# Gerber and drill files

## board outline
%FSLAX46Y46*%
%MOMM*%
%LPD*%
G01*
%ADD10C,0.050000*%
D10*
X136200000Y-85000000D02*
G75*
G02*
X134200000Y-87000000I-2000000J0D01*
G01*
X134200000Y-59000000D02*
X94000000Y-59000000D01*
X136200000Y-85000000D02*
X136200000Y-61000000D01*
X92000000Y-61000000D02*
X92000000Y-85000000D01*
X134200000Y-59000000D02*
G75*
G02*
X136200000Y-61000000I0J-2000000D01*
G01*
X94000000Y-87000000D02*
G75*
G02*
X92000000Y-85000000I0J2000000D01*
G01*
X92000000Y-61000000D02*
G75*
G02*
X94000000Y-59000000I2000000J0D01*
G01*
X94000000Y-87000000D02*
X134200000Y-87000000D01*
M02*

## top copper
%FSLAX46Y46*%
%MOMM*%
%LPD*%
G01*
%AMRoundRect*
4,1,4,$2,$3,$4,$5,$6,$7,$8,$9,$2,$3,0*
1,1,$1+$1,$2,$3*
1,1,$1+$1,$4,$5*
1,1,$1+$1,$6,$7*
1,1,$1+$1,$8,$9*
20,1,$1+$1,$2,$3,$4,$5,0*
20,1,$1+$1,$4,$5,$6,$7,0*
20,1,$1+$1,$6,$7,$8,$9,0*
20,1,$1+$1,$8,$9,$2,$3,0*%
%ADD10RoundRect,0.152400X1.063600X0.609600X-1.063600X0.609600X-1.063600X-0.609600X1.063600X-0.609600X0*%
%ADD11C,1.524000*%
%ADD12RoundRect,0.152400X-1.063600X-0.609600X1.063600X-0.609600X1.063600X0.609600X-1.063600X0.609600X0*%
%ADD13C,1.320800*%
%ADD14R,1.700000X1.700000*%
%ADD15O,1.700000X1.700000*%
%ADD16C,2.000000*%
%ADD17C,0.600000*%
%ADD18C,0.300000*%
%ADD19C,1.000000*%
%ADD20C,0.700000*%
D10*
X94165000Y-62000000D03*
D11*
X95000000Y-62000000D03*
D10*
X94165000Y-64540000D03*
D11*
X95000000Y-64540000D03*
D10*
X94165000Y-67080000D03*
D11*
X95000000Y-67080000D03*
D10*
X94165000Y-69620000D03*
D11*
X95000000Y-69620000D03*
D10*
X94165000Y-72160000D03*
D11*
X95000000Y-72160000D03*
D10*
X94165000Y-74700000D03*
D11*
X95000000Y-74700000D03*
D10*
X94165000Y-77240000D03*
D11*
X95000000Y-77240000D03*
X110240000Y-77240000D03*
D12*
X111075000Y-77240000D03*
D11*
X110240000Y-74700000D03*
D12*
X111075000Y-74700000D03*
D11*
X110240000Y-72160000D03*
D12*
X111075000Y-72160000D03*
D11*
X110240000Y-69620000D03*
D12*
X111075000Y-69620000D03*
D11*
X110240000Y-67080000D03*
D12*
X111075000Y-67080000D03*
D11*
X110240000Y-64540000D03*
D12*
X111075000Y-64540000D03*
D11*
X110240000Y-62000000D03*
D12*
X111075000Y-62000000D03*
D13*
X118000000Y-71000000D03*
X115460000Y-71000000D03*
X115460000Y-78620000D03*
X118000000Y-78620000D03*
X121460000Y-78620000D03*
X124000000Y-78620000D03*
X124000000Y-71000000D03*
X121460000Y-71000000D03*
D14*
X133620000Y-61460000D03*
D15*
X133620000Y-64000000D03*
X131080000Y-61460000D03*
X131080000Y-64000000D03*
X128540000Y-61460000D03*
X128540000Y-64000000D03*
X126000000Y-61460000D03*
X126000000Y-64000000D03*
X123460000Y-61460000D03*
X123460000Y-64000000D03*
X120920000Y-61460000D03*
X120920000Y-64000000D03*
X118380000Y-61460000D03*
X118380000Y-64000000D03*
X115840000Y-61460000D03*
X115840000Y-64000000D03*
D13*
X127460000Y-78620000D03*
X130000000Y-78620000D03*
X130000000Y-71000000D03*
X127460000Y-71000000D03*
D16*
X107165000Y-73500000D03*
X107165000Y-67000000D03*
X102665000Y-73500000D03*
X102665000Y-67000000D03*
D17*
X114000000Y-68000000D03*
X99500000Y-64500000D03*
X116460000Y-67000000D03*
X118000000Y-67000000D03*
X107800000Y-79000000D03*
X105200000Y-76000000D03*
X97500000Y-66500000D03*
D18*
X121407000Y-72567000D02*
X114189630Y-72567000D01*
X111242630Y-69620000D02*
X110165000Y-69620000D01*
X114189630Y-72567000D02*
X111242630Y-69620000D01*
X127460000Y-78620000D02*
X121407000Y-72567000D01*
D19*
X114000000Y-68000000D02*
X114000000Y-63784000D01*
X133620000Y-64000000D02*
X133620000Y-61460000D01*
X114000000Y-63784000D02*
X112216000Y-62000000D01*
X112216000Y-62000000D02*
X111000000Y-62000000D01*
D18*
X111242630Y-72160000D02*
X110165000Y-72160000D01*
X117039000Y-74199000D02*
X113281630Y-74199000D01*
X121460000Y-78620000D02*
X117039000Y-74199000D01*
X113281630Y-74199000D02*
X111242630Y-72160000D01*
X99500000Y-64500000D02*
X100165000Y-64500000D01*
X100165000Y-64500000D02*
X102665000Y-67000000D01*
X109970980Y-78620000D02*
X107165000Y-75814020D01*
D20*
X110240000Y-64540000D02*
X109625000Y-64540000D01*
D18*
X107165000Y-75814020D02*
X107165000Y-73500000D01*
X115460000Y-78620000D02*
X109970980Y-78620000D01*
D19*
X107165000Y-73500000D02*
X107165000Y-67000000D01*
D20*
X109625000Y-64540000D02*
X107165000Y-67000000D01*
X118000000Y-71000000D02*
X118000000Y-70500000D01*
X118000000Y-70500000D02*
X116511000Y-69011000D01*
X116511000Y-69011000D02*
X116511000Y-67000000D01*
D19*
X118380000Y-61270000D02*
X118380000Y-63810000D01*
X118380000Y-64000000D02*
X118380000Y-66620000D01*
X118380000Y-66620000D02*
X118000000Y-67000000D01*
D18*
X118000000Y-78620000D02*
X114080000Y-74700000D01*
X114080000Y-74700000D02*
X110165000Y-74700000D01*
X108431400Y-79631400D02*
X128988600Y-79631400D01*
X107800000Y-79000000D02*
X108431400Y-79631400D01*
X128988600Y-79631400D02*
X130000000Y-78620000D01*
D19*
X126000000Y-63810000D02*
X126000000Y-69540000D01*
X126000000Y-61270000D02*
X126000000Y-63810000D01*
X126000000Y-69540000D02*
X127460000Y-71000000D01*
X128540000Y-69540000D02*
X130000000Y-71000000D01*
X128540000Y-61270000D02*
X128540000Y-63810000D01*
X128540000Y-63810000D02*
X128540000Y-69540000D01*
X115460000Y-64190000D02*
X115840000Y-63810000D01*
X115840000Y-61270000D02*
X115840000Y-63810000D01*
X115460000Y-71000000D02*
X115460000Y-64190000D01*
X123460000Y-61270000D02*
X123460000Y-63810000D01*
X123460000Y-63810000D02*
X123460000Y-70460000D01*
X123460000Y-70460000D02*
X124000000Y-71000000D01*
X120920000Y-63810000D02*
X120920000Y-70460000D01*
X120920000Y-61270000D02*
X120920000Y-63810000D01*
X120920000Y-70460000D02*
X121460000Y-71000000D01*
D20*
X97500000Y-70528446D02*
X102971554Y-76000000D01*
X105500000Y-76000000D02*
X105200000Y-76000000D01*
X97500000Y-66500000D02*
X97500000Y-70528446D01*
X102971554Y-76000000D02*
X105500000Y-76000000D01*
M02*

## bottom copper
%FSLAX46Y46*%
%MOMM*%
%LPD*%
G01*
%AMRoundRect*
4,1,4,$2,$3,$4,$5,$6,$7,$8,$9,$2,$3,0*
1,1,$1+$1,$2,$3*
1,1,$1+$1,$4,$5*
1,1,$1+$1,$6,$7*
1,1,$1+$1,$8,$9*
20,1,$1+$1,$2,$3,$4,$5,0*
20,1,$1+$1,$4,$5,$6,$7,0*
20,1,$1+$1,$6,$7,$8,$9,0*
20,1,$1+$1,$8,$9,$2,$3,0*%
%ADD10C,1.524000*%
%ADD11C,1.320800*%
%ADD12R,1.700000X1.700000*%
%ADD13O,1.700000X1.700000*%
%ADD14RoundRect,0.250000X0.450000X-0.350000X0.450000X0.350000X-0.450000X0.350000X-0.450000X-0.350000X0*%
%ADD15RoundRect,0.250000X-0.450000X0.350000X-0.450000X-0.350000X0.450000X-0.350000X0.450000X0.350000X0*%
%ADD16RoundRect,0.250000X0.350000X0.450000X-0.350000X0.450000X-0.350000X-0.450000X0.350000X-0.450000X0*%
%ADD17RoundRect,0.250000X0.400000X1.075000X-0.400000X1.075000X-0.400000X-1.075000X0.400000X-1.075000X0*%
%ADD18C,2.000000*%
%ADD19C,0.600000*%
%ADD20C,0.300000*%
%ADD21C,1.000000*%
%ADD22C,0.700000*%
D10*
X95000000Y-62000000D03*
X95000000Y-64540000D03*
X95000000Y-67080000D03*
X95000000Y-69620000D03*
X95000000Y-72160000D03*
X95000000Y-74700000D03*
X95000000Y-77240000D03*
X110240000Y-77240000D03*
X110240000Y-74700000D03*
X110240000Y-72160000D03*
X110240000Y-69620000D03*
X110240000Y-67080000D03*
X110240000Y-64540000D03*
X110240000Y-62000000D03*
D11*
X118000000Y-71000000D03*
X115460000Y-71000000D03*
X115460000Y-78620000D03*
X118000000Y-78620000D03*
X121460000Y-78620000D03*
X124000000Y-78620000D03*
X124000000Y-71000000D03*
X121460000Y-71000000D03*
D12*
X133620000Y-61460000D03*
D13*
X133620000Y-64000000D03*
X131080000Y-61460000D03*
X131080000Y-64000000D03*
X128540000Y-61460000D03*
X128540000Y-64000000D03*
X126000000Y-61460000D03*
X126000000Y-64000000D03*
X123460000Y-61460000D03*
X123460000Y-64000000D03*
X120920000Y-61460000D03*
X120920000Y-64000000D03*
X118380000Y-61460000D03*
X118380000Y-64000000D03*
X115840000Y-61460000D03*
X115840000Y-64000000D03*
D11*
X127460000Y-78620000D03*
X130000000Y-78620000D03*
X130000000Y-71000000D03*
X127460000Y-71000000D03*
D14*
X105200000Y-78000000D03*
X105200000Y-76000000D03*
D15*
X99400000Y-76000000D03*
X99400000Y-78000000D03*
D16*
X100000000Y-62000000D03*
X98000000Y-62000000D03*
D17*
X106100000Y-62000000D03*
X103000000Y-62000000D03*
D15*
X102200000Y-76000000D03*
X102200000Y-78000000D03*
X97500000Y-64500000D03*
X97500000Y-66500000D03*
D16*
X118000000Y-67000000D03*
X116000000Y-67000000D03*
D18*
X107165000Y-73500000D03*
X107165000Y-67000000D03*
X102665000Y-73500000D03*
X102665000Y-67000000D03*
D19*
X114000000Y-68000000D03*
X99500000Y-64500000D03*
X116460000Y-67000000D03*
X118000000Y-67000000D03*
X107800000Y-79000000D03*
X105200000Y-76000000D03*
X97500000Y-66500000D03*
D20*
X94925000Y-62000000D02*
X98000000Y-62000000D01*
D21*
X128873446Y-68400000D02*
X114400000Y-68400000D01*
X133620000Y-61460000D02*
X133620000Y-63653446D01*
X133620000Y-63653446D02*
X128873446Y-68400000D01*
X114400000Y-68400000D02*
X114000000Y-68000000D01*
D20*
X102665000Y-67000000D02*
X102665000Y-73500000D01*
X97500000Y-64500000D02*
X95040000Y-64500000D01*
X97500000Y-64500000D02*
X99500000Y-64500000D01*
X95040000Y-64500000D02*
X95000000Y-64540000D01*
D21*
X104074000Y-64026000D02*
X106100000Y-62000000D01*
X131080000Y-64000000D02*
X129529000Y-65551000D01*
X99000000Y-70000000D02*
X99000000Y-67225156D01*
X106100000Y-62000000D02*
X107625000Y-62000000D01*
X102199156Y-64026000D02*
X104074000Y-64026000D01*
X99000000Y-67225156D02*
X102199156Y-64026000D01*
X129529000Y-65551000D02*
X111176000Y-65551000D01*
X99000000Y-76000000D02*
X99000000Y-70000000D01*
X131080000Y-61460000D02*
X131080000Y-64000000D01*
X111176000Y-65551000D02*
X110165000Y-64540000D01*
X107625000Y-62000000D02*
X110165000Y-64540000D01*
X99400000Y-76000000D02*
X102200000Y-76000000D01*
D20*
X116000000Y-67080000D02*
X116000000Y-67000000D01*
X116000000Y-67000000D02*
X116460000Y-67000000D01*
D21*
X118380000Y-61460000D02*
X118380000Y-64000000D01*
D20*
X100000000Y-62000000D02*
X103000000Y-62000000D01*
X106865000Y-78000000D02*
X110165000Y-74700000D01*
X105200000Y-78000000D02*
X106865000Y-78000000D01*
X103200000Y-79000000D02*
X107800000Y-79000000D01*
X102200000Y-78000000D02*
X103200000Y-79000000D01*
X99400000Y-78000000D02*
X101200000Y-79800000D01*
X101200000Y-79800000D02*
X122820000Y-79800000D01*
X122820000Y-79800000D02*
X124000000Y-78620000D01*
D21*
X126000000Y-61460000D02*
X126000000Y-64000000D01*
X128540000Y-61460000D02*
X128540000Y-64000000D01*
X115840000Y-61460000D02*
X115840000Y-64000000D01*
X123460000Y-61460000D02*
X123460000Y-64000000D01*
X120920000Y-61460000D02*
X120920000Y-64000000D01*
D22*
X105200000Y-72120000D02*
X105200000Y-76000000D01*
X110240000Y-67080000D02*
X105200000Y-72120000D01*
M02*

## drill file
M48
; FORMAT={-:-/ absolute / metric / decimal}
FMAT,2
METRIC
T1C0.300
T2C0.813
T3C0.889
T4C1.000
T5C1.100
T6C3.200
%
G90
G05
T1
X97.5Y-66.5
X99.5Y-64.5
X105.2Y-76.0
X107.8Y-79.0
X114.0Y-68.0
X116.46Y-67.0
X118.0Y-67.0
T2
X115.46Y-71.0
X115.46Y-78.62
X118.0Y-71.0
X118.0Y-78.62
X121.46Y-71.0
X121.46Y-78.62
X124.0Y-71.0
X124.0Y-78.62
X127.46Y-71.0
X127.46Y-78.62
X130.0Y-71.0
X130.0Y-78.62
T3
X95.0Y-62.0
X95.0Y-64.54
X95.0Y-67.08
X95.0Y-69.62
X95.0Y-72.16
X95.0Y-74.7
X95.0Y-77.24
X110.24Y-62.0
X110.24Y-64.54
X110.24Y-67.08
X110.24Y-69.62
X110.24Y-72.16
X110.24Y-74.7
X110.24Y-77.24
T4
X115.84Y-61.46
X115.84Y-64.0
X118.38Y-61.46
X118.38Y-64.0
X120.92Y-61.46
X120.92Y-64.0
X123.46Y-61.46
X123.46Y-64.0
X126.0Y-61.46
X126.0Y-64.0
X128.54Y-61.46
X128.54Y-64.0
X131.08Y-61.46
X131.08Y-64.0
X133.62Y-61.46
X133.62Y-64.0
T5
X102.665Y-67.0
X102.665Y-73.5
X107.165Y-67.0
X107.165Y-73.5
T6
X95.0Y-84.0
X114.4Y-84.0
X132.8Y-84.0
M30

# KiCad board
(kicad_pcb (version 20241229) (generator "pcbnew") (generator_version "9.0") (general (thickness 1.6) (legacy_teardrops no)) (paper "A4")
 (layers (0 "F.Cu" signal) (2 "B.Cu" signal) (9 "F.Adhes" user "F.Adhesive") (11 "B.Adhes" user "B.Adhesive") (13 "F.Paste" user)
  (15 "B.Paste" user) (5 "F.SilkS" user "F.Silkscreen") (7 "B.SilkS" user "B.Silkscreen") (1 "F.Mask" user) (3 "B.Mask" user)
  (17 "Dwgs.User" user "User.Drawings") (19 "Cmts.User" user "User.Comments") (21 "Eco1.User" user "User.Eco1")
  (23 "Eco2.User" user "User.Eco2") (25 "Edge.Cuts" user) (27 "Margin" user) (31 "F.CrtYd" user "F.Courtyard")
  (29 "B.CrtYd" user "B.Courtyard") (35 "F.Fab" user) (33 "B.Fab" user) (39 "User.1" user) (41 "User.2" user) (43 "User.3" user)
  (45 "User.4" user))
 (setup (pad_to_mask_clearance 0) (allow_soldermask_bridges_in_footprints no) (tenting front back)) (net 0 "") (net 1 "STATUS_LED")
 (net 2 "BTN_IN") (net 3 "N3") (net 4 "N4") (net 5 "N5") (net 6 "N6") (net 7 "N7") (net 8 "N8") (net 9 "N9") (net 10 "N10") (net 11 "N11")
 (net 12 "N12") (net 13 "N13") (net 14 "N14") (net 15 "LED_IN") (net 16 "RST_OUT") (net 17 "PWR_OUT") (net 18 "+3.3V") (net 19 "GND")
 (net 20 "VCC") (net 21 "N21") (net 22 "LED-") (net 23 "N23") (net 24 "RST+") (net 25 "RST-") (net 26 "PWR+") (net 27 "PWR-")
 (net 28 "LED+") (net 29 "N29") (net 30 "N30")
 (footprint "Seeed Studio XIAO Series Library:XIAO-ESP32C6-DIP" (layer "F.Cu") (at 102.665 69.62)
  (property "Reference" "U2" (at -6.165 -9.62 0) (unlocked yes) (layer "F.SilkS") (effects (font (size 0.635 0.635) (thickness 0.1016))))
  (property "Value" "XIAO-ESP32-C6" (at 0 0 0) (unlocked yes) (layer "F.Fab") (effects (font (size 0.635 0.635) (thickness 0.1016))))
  (pad "1" smd roundrect (at -8.5 -7.62 180) (size 2.432 1.524) (layers "F.Cu" "F.Mask") (roundrect_rratio 0.1) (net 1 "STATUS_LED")
   (thermal_bridge_angle 45))
  (pad "1" thru_hole circle (at -7.665 -7.62 180) (size 1.524 1.524) (drill 0.889) (layers "*.Cu" "*.Mask") (remove_unused_layers no)
   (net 1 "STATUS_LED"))
  (pad "2" smd roundrect (at -8.5 -5.08 180) (size 2.432 1.524) (layers "F.Cu" "F.Mask") (roundrect_rratio 0.1) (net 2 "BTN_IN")
   (thermal_bridge_angle 45))
  (pad "2" thru_hole circle (at -7.665 -5.08 180) (size 1.524 1.524) (drill 0.889) (layers "*.Cu" "*.Mask") (remove_unused_layers no)
   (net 2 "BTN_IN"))
  (pad "3" smd roundrect (at -8.5 -2.54 180) (size 2.432 1.524) (layers "F.Cu" "F.Mask") (roundrect_rratio 0.1) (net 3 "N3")
   (thermal_bridge_angle 45))
  (pad "3" thru_hole circle (at -7.665 -2.54 180) (size 1.524 1.524) (drill 0.889) (layers "*.Cu" "*.Mask") (remove_unused_layers no)
   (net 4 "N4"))
  (pad "4" smd roundrect (at -8.5 0 180) (size 2.432 1.524) (layers "F.Cu" "F.Mask") (roundrect_rratio 0.1) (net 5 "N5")
   (thermal_bridge_angle 45))
  (pad "4" thru_hole circle (at -7.665 0 180) (size 1.524 1.524) (drill 0.889) (layers "*.Cu" "*.Mask") (remove_unused_layers no)
   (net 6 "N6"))
  (pad "5" smd roundrect (at -8.5 2.54 180) (size 2.432 1.524) (layers "F.Cu" "F.Mask") (roundrect_rratio 0.1) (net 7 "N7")
   (thermal_bridge_angle 45))
  (pad "5" thru_hole circle (at -7.665 2.54 180) (size 1.524 1.524) (drill 0.889) (layers "*.Cu" "*.Mask") (remove_unused_layers no)
   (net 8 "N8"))
  (pad "6" smd roundrect (at -8.5 5.08 180) (size 2.432 1.524) (layers "F.Cu" "F.Mask") (roundrect_rratio 0.1) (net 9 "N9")
   (thermal_bridge_angle 45))
  (pad "6" thru_hole circle (at -7.665 5.08 180) (size 1.524 1.524) (drill 0.889) (layers "*.Cu" "*.Mask") (remove_unused_layers no)
   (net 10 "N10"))
  (pad "7" smd roundrect (at -8.5 7.62 180) (size 2.432 1.524) (layers "F.Cu" "F.Mask") (roundrect_rratio 0.1) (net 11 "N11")
   (thermal_bridge_angle 45))
  (pad "7" thru_hole circle (at -7.665 7.62 180) (size 1.524 1.524) (drill 0.889) (layers "*.Cu" "*.Mask") (remove_unused_layers no)
   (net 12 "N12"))
  (pad "8" thru_hole circle (at 7.575 7.62) (size 1.524 1.524) (drill 0.889) (layers "*.Cu" "*.Mask") (remove_unused_layers no)
   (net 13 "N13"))
  (pad "8" smd roundrect (at 8.41 7.62) (size 2.432 1.524) (layers "F.Cu" "F.Mask") (roundrect_rratio 0.1) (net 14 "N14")
   (thermal_bridge_angle 45))
  (pad "9" thru_hole circle (at 7.575 5.08) (size 1.524 1.524) (drill 0.889) (layers "*.Cu" "*.Mask") (remove_unused_layers no)
   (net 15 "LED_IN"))
  (pad "9" smd roundrect (at 8.41 5.08) (size 2.432 1.524) (layers "F.Cu" "F.Mask") (roundrect_rratio 0.1) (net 15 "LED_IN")
   (thermal_bridge_angle 45))
  (pad "10" thru_hole circle (at 7.575 2.54) (size 1.524 1.524) (drill 0.889) (layers "*.Cu" "*.Mask") (remove_unused_layers no)
   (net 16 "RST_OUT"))
  (pad "10" smd roundrect (at 8.41 2.54) (size 2.432 1.524) (layers "F.Cu" "F.Mask") (roundrect_rratio 0.1) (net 16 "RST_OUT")
   (thermal_bridge_angle 45))
  (pad "11" thru_hole circle (at 7.575 0) (size 1.524 1.524) (drill 0.889) (layers "*.Cu" "*.Mask") (remove_unused_layers no)
   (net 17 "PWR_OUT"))
  (pad "11" smd roundrect (at 8.41 0) (size 2.432 1.524) (layers "F.Cu" "F.Mask") (roundrect_rratio 0.1) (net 17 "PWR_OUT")
   (thermal_bridge_angle 45))
  (pad "12" thru_hole circle (at 7.575 -2.54) (size 1.524 1.524) (drill 0.889) (layers "*.Cu" "*.Mask") (remove_unused_layers no)
   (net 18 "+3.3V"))
  (pad "12" smd roundrect (at 8.41 -2.54) (size 2.432 1.524) (layers "F.Cu" "F.Mask") (roundrect_rratio 0.1) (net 18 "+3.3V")
   (thermal_bridge_angle 45))
  (pad "13" thru_hole circle (at 7.575 -5.08) (size 1.524 1.524) (drill 0.889) (layers "*.Cu" "*.Mask") (remove_unused_layers no)
   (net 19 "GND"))
  (pad "13" smd roundrect (at 8.41 -5.08) (size 2.432 1.524) (layers "F.Cu" "F.Mask") (roundrect_rratio 0.1) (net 19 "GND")
   (thermal_bridge_angle 45))
  (pad "14" thru_hole circle (at 7.575 -7.62) (size 1.524 1.524) (drill 0.889) (layers "*.Cu" "*.Mask") (remove_unused_layers no)
   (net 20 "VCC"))
  (pad "14" smd roundrect (at 8.41 -7.62) (size 2.432 1.524) (layers "F.Cu" "F.Mask") (roundrect_rratio 0.1) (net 20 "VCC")
   (thermal_bridge_angle 45)))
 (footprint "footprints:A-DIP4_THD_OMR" (layer "F.Cu") (at 118 71 -90)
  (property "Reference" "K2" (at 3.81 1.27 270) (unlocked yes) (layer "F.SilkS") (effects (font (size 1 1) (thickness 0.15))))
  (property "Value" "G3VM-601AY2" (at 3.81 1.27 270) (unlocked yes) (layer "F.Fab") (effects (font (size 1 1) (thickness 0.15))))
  (pad "1" thru_hole circle (at 0 0 270) (size 1.3208 1.3208) (drill 0.8128) (layers "*.Cu" "*.Mask") (remove_unused_layers no)
   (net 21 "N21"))
  (pad "2" thru_hole circle (at 0 2.54 270) (size 1.3208 1.3208) (drill 0.8128) (layers "*.Cu" "*.Mask") (remove_unused_layers no)
   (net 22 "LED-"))
  (pad "3" thru_hole circle (at 7.62 2.54 270) (size 1.3208 1.3208) (drill 0.8128) (layers "*.Cu" "*.Mask") (remove_unused_layers no)
   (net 19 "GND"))
  (pad "4" thru_hole circle (at 7.62 0 270) (size 1.3208 1.3208) (drill 0.8128) (layers "*.Cu" "*.Mask") (remove_unused_layers no)
   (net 15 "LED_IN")))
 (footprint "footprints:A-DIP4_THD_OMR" (layer "F.Cu") (at 121.46 78.62 90)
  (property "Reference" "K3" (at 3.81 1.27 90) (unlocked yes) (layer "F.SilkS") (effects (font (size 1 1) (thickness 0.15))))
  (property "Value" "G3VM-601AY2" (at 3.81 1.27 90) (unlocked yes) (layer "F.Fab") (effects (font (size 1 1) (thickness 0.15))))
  (pad "1" thru_hole circle (at 0 0 90) (size 1.3208 1.3208) (drill 0.8128) (layers "*.Cu" "*.Mask") (remove_unused_layers no)
   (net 16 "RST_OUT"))
  (pad "2" thru_hole circle (at 0 2.54 90) (size 1.3208 1.3208) (drill 0.8128) (layers "*.Cu" "*.Mask") (remove_unused_layers no)
   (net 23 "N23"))
  (pad "3" thru_hole circle (at 7.62 2.54 90) (size 1.3208 1.3208) (drill 0.8128) (layers "*.Cu" "*.Mask") (remove_unused_layers no)
   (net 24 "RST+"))
  (pad "4" thru_hole circle (at 7.62 0 90) (size 1.3208 1.3208) (drill 0.8128) (layers "*.Cu" "*.Mask") (remove_unused_layers no)
   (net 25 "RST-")))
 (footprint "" (layer "F.Cu") (at 132.8 84)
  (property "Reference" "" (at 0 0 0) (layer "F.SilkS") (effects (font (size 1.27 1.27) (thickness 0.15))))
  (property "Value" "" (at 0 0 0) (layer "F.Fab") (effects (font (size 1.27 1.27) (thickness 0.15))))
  (pad "" np_thru_hole circle (at 0 0) (size 3.2 3.2) (drill 3.2) (layers "*.Cu" "*.Mask")))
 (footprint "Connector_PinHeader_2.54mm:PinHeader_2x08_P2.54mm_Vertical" (layer "F.Cu") (at 133.62 61.46 -90)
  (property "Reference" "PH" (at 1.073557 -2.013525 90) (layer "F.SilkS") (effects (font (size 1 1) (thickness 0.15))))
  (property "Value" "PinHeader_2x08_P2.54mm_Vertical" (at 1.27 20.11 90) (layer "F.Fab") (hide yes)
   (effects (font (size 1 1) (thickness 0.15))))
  (pad "1" thru_hole rect (at 0 0 270) (size 1.7 1.7) (drill 1) (layers "*.Cu" "*.Mask") (remove_unused_layers no) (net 20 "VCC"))
  (pad "2" thru_hole oval (at 2.54 0 270) (size 1.7 1.7) (drill 1) (layers "*.Cu" "*.Mask") (remove_unused_layers no) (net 20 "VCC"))
  (pad "3" thru_hole oval (at 0 2.54 270) (size 1.7 1.7) (drill 1) (layers "*.Cu" "*.Mask") (remove_unused_layers no) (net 19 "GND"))
  (pad "4" thru_hole oval (at 2.54 2.54 270) (size 1.7 1.7) (drill 1) (layers "*.Cu" "*.Mask") (remove_unused_layers no) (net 19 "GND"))
  (pad "5" thru_hole oval (at 0 5.08 270) (size 1.7 1.7) (drill 1) (layers "*.Cu" "*.Mask") (remove_unused_layers no) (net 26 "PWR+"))
  (pad "6" thru_hole oval (at 2.54 5.08 270) (size 1.7 1.7) (drill 1) (layers "*.Cu" "*.Mask") (remove_unused_layers no) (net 26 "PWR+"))
  (pad "7" thru_hole oval (at 0 7.62 270) (size 1.7 1.7) (drill 1) (layers "*.Cu" "*.Mask") (remove_unused_layers no) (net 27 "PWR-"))
  (pad "8" thru_hole oval (at 2.54 7.62 270) (size 1.7 1.7) (drill 1) (layers "*.Cu" "*.Mask") (remove_unused_layers no) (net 27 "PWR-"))
  (pad "9" thru_hole oval (at 0 10.16 270) (size 1.7 1.7) (drill 1) (layers "*.Cu" "*.Mask") (remove_unused_layers no) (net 24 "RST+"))
  (pad "10" thru_hole oval (at 2.54 10.16 270) (size 1.7 1.7) (drill 1) (layers "*.Cu" "*.Mask") (remove_unused_layers no) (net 24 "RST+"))
  (pad "11" thru_hole oval (at 0 12.7 270) (size 1.7 1.7) (drill 1) (layers "*.Cu" "*.Mask") (remove_unused_layers no) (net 25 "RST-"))
  (pad "12" thru_hole oval (at 2.54 12.7 270) (size 1.7 1.7) (drill 1) (layers "*.Cu" "*.Mask") (remove_unused_layers no) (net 25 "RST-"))
  (pad "13" thru_hole oval (at 0 15.24 270) (size 1.7 1.7) (drill 1) (layers "*.Cu" "*.Mask") (remove_unused_layers no) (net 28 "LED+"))
  (pad "14" thru_hole oval (at 2.54 15.24 270) (size 1.7 1.7) (drill 1) (layers "*.Cu" "*.Mask") (remove_unused_layers no) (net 28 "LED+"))
  (pad "15" thru_hole oval (at 0 17.78 270) (size 1.7 1.7) (drill 1) (layers "*.Cu" "*.Mask") (remove_unused_layers no) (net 22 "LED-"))
  (pad "16" thru_hole oval (at 2.54 17.78 270) (size 1.7 1.7) (drill 1) (layers "*.Cu" "*.Mask") (remove_unused_layers no) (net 22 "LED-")))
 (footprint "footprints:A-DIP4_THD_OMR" (layer "F.Cu") (at 127.46 78.62 90)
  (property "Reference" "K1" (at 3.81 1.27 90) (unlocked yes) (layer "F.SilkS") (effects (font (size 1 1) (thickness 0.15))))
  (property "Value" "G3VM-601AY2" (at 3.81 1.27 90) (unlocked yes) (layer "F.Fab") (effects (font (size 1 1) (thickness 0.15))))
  (pad "1" thru_hole circle (at 0 0 90) (size 1.3208 1.3208) (drill 0.8128) (layers "*.Cu" "*.Mask") (remove_unused_layers no)
   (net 17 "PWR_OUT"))
  (pad "2" thru_hole circle (at 0 2.54 90) (size 1.3208 1.3208) (drill 0.8128) (layers "*.Cu" "*.Mask") (remove_unused_layers no)
   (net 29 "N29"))
  (pad "3" thru_hole circle (at 7.62 2.54 90) (size 1.3208 1.3208) (drill 0.8128) (layers "*.Cu" "*.Mask") (remove_unused_layers no)
   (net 26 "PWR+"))
  (pad "4" thru_hole circle (at 7.62 0 90) (size 1.3208 1.3208) (drill 0.8128) (layers "*.Cu" "*.Mask") (remove_unused_layers no)
   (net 27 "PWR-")))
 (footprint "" (layer "F.Cu") (at 114.4 84)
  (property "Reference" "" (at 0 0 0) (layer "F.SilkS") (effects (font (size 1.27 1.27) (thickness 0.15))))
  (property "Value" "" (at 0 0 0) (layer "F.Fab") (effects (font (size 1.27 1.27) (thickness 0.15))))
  (pad "" np_thru_hole circle (at 0 0) (size 3.2 3.2) (drill 3.2) (layers "*.Cu" "*.Mask")))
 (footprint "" (layer "F.Cu") (at 95 84)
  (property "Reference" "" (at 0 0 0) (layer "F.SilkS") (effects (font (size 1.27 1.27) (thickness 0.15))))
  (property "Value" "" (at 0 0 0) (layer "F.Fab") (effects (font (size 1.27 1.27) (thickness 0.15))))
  (pad "" np_thru_hole circle (at 0 0) (size 3.2 3.2) (drill 3.2) (layers "*.Cu" "*.Mask")))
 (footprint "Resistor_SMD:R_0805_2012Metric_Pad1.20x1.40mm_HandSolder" (layer "B.Cu") (at 105.2 77 90)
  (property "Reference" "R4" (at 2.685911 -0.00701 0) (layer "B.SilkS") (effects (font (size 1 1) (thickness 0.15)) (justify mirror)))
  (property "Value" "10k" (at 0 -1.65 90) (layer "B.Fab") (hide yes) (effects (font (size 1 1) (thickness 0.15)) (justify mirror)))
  (pad "1" smd roundrect (at -1 0 90) (size 1.2 1.4) (layers "B.Cu" "B.Mask" "B.Paste") (roundrect_rratio 0.208333) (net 15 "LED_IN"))
  (pad "2" smd roundrect (at 1 0 90) (size 1.2 1.4) (layers "B.Cu" "B.Mask" "B.Paste") (roundrect_rratio 0.208333) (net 18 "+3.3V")))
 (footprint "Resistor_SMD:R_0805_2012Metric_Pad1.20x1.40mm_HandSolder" (layer "B.Cu") (at 99.4 77 -90)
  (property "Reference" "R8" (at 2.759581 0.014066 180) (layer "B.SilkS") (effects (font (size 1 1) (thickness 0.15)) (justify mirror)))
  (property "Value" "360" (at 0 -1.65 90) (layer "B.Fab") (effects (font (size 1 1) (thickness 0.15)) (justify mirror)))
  (pad "1" smd roundrect (at -1 0 270) (size 1.2 1.4) (layers "B.Cu" "B.Mask" "B.Paste") (roundrect_rratio 0.208333) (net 19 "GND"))
  (pad "2" smd roundrect (at 1 0 270) (size 1.2 1.4) (layers "B.Cu" "B.Mask" "B.Paste") (roundrect_rratio 0.208333) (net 23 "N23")))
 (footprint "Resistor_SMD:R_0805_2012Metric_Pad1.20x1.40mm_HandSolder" (layer "B.Cu") (at 99 62 180)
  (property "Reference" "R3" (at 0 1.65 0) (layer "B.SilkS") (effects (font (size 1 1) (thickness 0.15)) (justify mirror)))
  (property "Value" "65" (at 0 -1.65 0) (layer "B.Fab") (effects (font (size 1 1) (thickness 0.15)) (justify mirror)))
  (pad "1" smd roundrect (at -1 0 180) (size 1.2 1.4) (layers "B.Cu" "B.Mask" "B.Paste") (roundrect_rratio 0.208333) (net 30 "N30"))
  (pad "2" smd roundrect (at 1 0 180) (size 1.2 1.4) (layers "B.Cu" "B.Mask" "B.Paste") (roundrect_rratio 0.208333) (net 1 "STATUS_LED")))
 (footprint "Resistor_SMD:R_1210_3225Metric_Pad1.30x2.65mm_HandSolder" (layer "B.Cu") (at 104.55 62 180)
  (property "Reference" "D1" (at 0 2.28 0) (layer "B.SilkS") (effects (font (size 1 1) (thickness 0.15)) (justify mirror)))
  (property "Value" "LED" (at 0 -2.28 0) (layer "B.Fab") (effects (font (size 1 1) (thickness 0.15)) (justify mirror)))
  (pad "1" smd roundrect (at -1.55 0 180) (size 1.3 2.65) (layers "B.Cu" "B.Mask" "B.Paste") (roundrect_rratio 0.192308) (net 19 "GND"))
  (pad "2" smd roundrect (at 1.55 0 180) (size 1.3 2.65) (layers "B.Cu" "B.Mask" "B.Paste") (roundrect_rratio 0.192308) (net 30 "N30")))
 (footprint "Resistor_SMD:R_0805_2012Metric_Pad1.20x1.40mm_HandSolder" (layer "B.Cu") (at 102.2 77 -90)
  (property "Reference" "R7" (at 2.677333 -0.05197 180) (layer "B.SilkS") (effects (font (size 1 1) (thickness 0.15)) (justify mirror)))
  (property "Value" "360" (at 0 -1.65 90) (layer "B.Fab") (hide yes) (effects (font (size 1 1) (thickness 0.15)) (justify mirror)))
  (pad "1" smd roundrect (at -1 0 270) (size 1.2 1.4) (layers "B.Cu" "B.Mask" "B.Paste") (roundrect_rratio 0.208333) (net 19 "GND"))
  (pad "2" smd roundrect (at 1 0 270) (size 1.2 1.4) (layers "B.Cu" "B.Mask" "B.Paste") (roundrect_rratio 0.208333) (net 29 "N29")))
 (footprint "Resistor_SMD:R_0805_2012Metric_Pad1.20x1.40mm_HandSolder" (layer "B.Cu") (at 97.5 65.5 -90)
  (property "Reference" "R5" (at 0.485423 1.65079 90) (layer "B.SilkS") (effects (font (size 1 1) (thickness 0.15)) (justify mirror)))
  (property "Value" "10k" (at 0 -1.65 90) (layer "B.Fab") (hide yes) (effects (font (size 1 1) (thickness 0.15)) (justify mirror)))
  (pad "1" smd roundrect (at -1 0 270) (size 1.2 1.4) (layers "B.Cu" "B.Mask" "B.Paste") (roundrect_rratio 0.208333) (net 2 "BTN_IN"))
  (pad "2" smd roundrect (at 1 0 270) (size 1.2 1.4) (layers "B.Cu" "B.Mask" "B.Paste") (roundrect_rratio 0.208333) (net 18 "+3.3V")))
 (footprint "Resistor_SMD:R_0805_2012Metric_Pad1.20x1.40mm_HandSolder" (layer "B.Cu") (at 117 67 180)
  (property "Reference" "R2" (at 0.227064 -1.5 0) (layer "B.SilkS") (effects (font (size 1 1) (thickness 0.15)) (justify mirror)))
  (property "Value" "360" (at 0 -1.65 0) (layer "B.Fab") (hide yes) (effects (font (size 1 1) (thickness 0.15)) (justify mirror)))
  (pad "1" smd roundrect (at -1 0 180) (size 1.2 1.4) (layers "B.Cu" "B.Mask" "B.Paste") (roundrect_rratio 0.208333) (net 28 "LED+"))
  (pad "2" smd roundrect (at 1 0 180) (size 1.2 1.4) (layers "B.Cu" "B.Mask" "B.Paste") (roundrect_rratio 0.208333) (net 21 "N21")))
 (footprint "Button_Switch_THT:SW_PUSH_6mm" (layer "B.Cu") (at 107.165 73.5 90)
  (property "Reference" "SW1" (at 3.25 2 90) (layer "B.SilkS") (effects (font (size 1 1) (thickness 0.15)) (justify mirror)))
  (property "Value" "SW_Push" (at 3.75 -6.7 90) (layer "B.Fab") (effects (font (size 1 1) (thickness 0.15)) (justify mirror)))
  (pad "1" thru_hole circle (at 0 0) (size 2 2) (drill 1.1) (layers "*.Cu" "*.Mask") (remove_unused_layers no) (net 19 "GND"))
  (pad "1" thru_hole circle (at 6.5 0) (size 2 2) (drill 1.1) (layers "*.Cu" "*.Mask") (remove_unused_layers no) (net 19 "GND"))
  (pad "2" thru_hole circle (at 0 -4.5) (size 2 2) (drill 1.1) (layers "*.Cu" "*.Mask") (remove_unused_layers no) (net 2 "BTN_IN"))
  (pad "2" thru_hole circle (at 6.5 -4.5) (size 2 2) (drill 1.1) (layers "*.Cu" "*.Mask") (remove_unused_layers no) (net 2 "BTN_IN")))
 (gr_arc (start 136.2 85) (mid 135.614214 86.414214) (end 134.2 87) (stroke (width 0.05) (type default)) (layer "Edge.Cuts"))
 (gr_line (start 134.2 59) (end 94 59) (stroke (width 0.05) (type default)) (layer "Edge.Cuts"))
 (gr_line (start 136.2 85) (end 136.2 61) (stroke (width 0.05) (type default)) (layer "Edge.Cuts"))
 (gr_line (start 92 61) (end 92 85) (stroke (width 0.05) (type default)) (layer "Edge.Cuts"))
 (gr_arc (start 134.2 59) (mid 135.614214 59.585786) (end 136.2 61) (stroke (width 0.05) (type default)) (layer "Edge.Cuts"))
 (gr_arc (start 94 87) (mid 92.585786 86.414214) (end 92 85) (stroke (width 0.05) (type default)) (layer "Edge.Cuts"))
 (gr_arc (start 92 61) (mid 92.585786 59.585786) (end 94 59) (stroke (width 0.05) (type default)) (layer "Edge.Cuts"))
 (gr_line (start 94 87) (end 134.2 87) (stroke (width 0.05) (type default)) (layer "Edge.Cuts"))
 (segment (start 121.407 72.567) (end 114.18963 72.567) (width 0.3) (layer "F.Cu") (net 17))
 (segment (start 111.24263 69.62) (end 110.165 69.62) (width 0.3) (layer "F.Cu") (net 17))
 (segment (start 114.18963 72.567) (end 111.24263 69.62) (width 0.3) (layer "F.Cu") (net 17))
 (segment (start 127.46 78.62) (end 121.407 72.567) (width 0.3) (layer "F.Cu") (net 17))
 (segment (start 94.925 62) (end 98 62) (width 0.3) (layer "B.Cu") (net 1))
 (segment (start 114 68) (end 114 63.784) (width 1) (layer "F.Cu") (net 20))
 (segment (start 133.62 64) (end 133.62 61.46) (width 1) (layer "F.Cu") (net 20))
 (segment (start 114 63.784) (end 112.216 62) (width 1) (layer "F.Cu") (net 20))
 (segment (start 112.216 62) (end 111 62) (width 1) (layer "F.Cu") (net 20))
 (via (at 114 68) (size 0.6) (drill 0.3) (layers "F.Cu" "B.Cu") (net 20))
 (segment (start 128.873446 68.4) (end 114.4 68.4) (width 1) (layer "B.Cu") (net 20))
 (segment (start 133.62 61.46) (end 133.62 63.653446) (width 1) (layer "B.Cu") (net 20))
 (segment (start 133.62 63.653446) (end 128.873446 68.4) (width 1) (layer "B.Cu") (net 20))
 (segment (start 114.4 68.4) (end 114 68) (width 1) (layer "B.Cu") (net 20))
 (segment (start 111.24263 72.16) (end 110.165 72.16) (width 0.3) (layer "F.Cu") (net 16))
 (segment (start 117.039 74.199) (end 113.28163 74.199) (width 0.3) (layer "F.Cu") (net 16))
 (segment (start 121.46 78.62) (end 117.039 74.199) (width 0.3) (layer "F.Cu") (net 16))
 (segment (start 113.28163 74.199) (end 111.24263 72.16) (width 0.3) (layer "F.Cu") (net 16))
 (segment (start 99.5 64.5) (end 100.165 64.5) (width 0.3) (layer "F.Cu") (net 2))
 (segment (start 100.165 64.5) (end 102.665 67) (width 0.3) (layer "F.Cu") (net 2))
 (via (at 99.5 64.5) (size 0.6) (drill 0.3) (layers "F.Cu" "B.Cu") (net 2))
 (segment (start 102.665 67) (end 102.665 73.5) (width 0.3) (layer "B.Cu") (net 2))
 (segment (start 97.5 64.5) (end 95.04 64.5) (width 0.3) (layer "B.Cu") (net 2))
 (segment (start 97.5 64.5) (end 99.5 64.5) (width 0.3) (layer "B.Cu") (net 2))
 (segment (start 95.04 64.5) (end 95 64.54) (width 0.3) (layer "B.Cu") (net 2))
 (segment (start 109.97098 78.62) (end 107.165 75.81402) (width 0.3) (layer "F.Cu") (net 19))
 (segment (start 110.24 64.54) (end 109.625 64.54) (width 0.7) (layer "F.Cu") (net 19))
 (segment (start 107.165 75.81402) (end 107.165 73.5) (width 0.3) (layer "F.Cu") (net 19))
 (segment (start 115.46 78.62) (end 109.97098 78.62) (width 0.3) (layer "F.Cu") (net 19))
 (segment (start 107.165 73.5) (end 107.165 67) (width 1) (layer "F.Cu") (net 19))
 (segment (start 109.625 64.54) (end 107.165 67) (width 0.7) (layer "F.Cu") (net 19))
 (segment (start 104.074 64.026) (end 106.1 62) (width 1) (layer "B.Cu") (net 19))
 (segment (start 131.08 64) (end 129.529 65.551) (width 1) (layer "B.Cu") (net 19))
 (segment (start 99 70) (end 99 67.225156) (width 1) (layer "B.Cu") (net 19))
 (segment (start 106.1 62) (end 107.625 62) (width 1) (layer "B.Cu") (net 19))
 (segment (start 102.199156 64.026) (end 104.074 64.026) (width 1) (layer "B.Cu") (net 19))
 (segment (start 99 67.225156) (end 102.199156 64.026) (width 1) (layer "B.Cu") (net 19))
 (segment (start 129.529 65.551) (end 111.176 65.551) (width 1) (layer "B.Cu") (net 19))
 (segment (start 99 76) (end 99 70) (width 1) (layer "B.Cu") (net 19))
 (segment (start 131.08 61.46) (end 131.08 64) (width 1) (layer "B.Cu") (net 19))
 (segment (start 111.176 65.551) (end 110.165 64.54) (width 1) (layer "B.Cu") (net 19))
 (segment (start 107.625 62) (end 110.165 64.54) (width 1) (layer "B.Cu") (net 19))
 (segment (start 99.4 76) (end 102.2 76) (width 1) (layer "B.Cu") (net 19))
 (segment (start 118 71) (end 118 70.5) (width 0.7) (layer "F.Cu") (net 21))
 (segment (start 118 70.5) (end 116.511 69.011) (width 0.7) (layer "F.Cu") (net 21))
 (segment (start 116.511 69.011) (end 116.511 67) (width 0.7) (layer "F.Cu") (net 21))
 (via (at 116.46 67) (size 0.6) (drill 0.3) (layers "F.Cu" "B.Cu") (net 21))
 (segment (start 116 67.08) (end 116 67) (width 0.3) (layer "B.Cu") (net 21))
 (segment (start 116 67) (end 116.46 67) (width 0.3) (layer "B.Cu") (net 21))
 (segment (start 118.38 61.27) (end 118.38 63.81) (width 1) (layer "F.Cu") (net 28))
 (segment (start 118.38 64) (end 118.38 66.62) (width 1) (layer "F.Cu") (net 28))
 (segment (start 118.38 66.62) (end 118 67) (width 1) (layer "F.Cu") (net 28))
 (via (at 118 67) (size 0.6) (drill 0.3) (layers "F.Cu" "B.Cu") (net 28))
 (segment (start 118.38 61.46) (end 118.38 64) (width 1) (layer "B.Cu") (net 28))
 (segment (start 100 62) (end 103 62) (width 0.3) (layer "B.Cu") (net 30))
 (segment (start 118 78.62) (end 114.08 74.7) (width 0.3) (layer "F.Cu") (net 15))
 (segment (start 114.08 74.7) (end 110.165 74.7) (width 0.3) (layer "F.Cu") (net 15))
 (segment (start 106.865 78) (end 110.165 74.7) (width 0.3) (layer "B.Cu") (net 15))
 (segment (start 105.2 78) (end 106.865 78) (width 0.3) (layer "B.Cu") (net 15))
 (segment (start 108.4314 79.6314) (end 128.9886 79.6314) (width 0.3) (layer "F.Cu") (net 29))
 (segment (start 107.8 79) (end 108.4314 79.6314) (width 0.3) (layer "F.Cu") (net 29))
 (segment (start 128.9886 79.6314) (end 130 78.62) (width 0.3) (layer "F.Cu") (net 29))
 (via (at 107.8 79) (size 0.6) (drill 0.3) (layers "F.Cu" "B.Cu") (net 29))
 (segment (start 103.2 79) (end 107.8 79) (width 0.3) (layer "B.Cu") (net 29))
 (segment (start 102.2 78) (end 103.2 79) (width 0.3) (layer "B.Cu") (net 29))
 (segment (start 99.4 78) (end 101.2 79.8) (width 0.3) (layer "B.Cu") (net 23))
 (segment (start 101.2 79.8) (end 122.82 79.8) (width 0.3) (layer "B.Cu") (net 23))
 (segment (start 122.82 79.8) (end 124 78.62) (width 0.3) (layer "B.Cu") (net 23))
 (segment (start 126 63.81) (end 126 69.54) (width 1) (layer "F.Cu") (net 27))
 (segment (start 126 61.27) (end 126 63.81) (width 1) (layer "F.Cu") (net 27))
 (segment (start 126 69.54) (end 127.46 71) (width 1) (layer "F.Cu") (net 27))
 (segment (start 126 61.46) (end 126 64) (width 1) (layer "B.Cu") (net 27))
 (segment (start 128.54 69.54) (end 130 71) (width 1) (layer "F.Cu") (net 26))
 (segment (start 128.54 61.27) (end 128.54 63.81) (width 1) (layer "F.Cu") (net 26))
 (segment (start 128.54 63.81) (end 128.54 69.54) (width 1) (layer "F.Cu") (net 26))
 (segment (start 128.54 61.46) (end 128.54 64) (width 1) (layer "B.Cu") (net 26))
 (segment (start 115.46 64.19) (end 115.84 63.81) (width 1) (layer "F.Cu") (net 22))
 (segment (start 115.84 61.27) (end 115.84 63.81) (width 1) (layer "F.Cu") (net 22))
 (segment (start 115.46 71) (end 115.46 64.19) (width 1) (layer "F.Cu") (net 22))
 (segment (start 115.84 61.46) (end 115.84 64) (width 1) (layer "B.Cu") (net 22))
 (segment (start 123.46 61.27) (end 123.46 63.81) (width 1) (layer "F.Cu") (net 24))
 (segment (start 123.46 63.81) (end 123.46 70.46) (width 1) (layer "F.Cu") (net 24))
 (segment (start 123.46 70.46) (end 124 71) (width 1) (layer "F.Cu") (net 24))
 (segment (start 123.46 61.46) (end 123.46 64) (width 1) (layer "B.Cu") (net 24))
 (segment (start 120.92 63.81) (end 120.92 70.46) (width 1) (layer "F.Cu") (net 25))
 (segment (start 120.92 61.27) (end 120.92 63.81) (width 1) (layer "F.Cu") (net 25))
 (segment (start 120.92 70.46) (end 121.46 71) (width 1) (layer "F.Cu") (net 25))
 (segment (start 120.92 61.46) (end 120.92 64) (width 1) (layer "B.Cu") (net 25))
 (segment (start 97.5 70.528446) (end 102.971554 76) (width 0.7) (layer "F.Cu") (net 18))
 (segment (start 105.5 76) (end 105.2 76) (width 0.7) (layer "F.Cu") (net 18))
 (segment (start 97.5 66.5) (end 97.5 70.528446) (width 0.7) (layer "F.Cu") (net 18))
 (segment (start 102.971554 76) (end 105.5 76) (width 0.7) (layer "F.Cu") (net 18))
 (via (at 105.2 76) (size 0.6) (drill 0.3) (layers "F.Cu" "B.Cu") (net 18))
 (via (at 97.5 66.5) (size 0.6) (drill 0.3) (layers "F.Cu" "B.Cu") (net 18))
 (segment (start 105.2 72.12) (end 105.2 76) (width 0.7) (layer "B.Cu") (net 18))
 (segment (start 110.24 67.08) (end 105.2 72.12) (width 0.7) (layer "B.Cu") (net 18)))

